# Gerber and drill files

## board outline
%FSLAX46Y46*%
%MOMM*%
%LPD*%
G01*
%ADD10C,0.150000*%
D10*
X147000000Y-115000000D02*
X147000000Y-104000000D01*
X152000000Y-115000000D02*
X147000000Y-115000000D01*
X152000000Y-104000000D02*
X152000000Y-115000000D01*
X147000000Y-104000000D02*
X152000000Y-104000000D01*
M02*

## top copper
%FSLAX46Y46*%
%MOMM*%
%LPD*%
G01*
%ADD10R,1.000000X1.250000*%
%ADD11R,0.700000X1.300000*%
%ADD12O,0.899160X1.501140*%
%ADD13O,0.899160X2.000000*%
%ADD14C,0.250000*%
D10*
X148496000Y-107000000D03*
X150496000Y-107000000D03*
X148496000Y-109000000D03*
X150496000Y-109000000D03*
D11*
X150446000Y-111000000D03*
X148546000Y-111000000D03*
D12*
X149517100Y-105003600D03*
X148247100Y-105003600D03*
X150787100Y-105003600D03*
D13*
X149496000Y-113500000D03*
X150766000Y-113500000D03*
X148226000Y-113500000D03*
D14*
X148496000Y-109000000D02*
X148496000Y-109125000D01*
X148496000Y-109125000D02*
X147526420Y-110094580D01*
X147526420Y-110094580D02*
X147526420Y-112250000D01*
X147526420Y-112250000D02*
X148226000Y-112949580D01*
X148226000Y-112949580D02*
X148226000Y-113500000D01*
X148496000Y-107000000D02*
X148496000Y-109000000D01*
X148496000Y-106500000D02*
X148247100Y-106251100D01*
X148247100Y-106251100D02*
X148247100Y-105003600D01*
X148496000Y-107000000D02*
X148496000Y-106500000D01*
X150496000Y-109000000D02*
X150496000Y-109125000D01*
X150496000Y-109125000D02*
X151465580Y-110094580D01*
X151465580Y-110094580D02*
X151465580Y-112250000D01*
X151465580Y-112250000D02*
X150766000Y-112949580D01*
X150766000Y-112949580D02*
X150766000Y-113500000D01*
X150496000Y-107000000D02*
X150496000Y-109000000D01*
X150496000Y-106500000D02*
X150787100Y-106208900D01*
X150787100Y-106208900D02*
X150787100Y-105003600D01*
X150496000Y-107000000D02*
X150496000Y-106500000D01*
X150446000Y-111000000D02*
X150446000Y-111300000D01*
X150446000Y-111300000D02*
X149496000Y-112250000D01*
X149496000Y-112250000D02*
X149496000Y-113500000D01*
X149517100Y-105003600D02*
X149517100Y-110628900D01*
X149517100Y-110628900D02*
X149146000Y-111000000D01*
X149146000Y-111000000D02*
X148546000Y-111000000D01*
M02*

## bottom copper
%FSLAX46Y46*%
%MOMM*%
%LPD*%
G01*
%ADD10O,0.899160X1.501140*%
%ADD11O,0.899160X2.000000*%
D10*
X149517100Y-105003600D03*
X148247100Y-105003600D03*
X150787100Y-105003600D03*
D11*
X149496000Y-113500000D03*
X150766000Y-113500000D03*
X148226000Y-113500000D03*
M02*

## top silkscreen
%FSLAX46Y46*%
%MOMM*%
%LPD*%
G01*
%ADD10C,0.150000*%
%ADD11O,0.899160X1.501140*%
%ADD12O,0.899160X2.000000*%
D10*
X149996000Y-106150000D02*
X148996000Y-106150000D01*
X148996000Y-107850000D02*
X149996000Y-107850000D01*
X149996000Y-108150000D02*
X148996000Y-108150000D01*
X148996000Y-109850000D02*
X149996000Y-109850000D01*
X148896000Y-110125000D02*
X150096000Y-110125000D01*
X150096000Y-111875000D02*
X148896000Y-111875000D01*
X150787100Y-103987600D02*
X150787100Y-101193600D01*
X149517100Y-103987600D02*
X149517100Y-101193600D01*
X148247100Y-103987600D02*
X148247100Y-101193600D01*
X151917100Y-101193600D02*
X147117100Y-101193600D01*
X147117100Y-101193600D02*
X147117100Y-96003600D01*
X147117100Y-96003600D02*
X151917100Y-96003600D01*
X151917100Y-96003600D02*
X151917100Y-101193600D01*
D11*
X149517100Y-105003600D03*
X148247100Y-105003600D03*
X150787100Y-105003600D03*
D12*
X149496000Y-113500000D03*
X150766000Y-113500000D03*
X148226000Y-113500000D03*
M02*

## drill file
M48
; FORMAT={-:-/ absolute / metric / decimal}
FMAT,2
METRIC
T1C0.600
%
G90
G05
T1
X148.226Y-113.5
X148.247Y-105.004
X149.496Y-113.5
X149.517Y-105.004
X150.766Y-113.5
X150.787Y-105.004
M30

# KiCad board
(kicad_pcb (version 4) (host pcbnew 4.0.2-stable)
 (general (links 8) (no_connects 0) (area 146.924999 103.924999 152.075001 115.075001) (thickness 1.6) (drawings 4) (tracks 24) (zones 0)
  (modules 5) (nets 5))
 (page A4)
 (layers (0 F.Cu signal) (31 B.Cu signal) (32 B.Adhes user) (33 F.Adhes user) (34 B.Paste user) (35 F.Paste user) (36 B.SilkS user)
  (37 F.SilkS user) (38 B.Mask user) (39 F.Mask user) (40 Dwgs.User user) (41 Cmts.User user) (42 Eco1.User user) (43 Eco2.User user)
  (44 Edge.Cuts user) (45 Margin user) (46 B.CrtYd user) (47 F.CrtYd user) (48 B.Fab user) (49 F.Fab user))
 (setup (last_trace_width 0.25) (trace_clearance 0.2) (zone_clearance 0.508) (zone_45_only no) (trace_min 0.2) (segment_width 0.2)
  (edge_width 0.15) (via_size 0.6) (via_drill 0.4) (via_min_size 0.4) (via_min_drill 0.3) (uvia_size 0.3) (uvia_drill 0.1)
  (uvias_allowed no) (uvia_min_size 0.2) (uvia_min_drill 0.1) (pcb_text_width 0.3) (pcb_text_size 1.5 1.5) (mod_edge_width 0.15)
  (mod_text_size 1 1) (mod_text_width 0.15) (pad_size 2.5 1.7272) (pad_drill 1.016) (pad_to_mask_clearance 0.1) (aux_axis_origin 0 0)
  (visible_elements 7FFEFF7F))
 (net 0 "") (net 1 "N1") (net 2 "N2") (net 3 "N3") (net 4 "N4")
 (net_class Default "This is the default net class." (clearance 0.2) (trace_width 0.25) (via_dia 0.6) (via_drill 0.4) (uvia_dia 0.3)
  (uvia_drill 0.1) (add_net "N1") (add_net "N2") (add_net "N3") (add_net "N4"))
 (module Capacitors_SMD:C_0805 (layer F.Cu) (at 149.496 107)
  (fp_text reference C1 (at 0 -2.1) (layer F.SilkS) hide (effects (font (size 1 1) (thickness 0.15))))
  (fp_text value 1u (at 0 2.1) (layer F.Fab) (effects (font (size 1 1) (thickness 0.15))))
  (fp_line (start 0.5 -0.85) (end -0.5 -0.85) (layer F.SilkS) (width 0.15))
  (fp_line (start -0.5 0.85) (end 0.5 0.85) (layer F.SilkS) (width 0.15))
  (pad 1 smd rect (at -1 0) (size 1 1.25) (layers F.Cu F.Paste F.Mask) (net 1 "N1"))
  (pad 2 smd rect (at 1 0) (size 1 1.25) (layers F.Cu F.Paste F.Mask) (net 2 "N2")))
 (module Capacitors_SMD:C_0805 (layer F.Cu) (at 149.496 109)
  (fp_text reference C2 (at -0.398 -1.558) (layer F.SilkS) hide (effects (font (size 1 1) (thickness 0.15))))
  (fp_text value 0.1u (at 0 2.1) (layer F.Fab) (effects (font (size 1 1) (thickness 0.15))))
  (fp_line (start 0.5 -0.85) (end -0.5 -0.85) (layer F.SilkS) (width 0.15))
  (fp_line (start -0.5 0.85) (end 0.5 0.85) (layer F.SilkS) (width 0.15))
  (pad 1 smd rect (at -1 0) (size 1 1.25) (layers F.Cu F.Paste F.Mask) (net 1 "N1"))
  (pad 2 smd rect (at 1 0) (size 1 1.25) (layers F.Cu F.Paste F.Mask) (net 2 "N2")))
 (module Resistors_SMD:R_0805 (layer F.Cu) (at 149.496 111 180)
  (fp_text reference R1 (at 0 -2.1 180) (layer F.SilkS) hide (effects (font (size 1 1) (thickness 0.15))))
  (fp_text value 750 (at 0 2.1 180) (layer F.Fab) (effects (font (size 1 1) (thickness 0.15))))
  (fp_line (start 0.6 0.875) (end -0.6 0.875) (layer F.SilkS) (width 0.15))
  (fp_line (start -0.6 -0.875) (end 0.6 -0.875) (layer F.SilkS) (width 0.15))
  (pad 1 smd rect (at -0.95 0 180) (size 0.7 1.3) (layers F.Cu F.Paste F.Mask) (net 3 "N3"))
  (pad 2 smd rect (at 0.95 0 180) (size 0.7 1.3) (layers F.Cu F.Paste F.Mask) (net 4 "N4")))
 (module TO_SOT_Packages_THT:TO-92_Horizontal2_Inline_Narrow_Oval (layer F.Cu) (at 148.2471 105.0036)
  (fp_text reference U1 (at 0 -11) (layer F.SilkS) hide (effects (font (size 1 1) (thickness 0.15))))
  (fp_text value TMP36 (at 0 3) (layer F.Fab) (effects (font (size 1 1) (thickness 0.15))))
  (fp_line (start 2.54 -1.016) (end 2.54 -3.81) (layer F.SilkS) (width 0.15))
  (fp_line (start 1.27 -1.016) (end 1.27 -3.81) (layer F.SilkS) (width 0.15))
  (fp_line (start 0 -1.016) (end 0 -3.81) (layer F.SilkS) (width 0.15))
  (fp_line (start 3.67 -3.81) (end -1.13 -3.81) (layer F.SilkS) (width 0.15))
  (fp_line (start -1.13 -3.81) (end -1.13 -9) (layer F.SilkS) (width 0.15))
  (fp_line (start -1.13 -9) (end 3.67 -9) (layer F.SilkS) (width 0.15))
  (fp_line (start 3.67 -9) (end 3.67 -3.81) (layer F.SilkS) (width 0.15))
  (pad 2 thru_hole oval (at 1.27 0) (size 0.89916 1.50114) (drill 0.6) (layers *.Cu *.Mask F.SilkS) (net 4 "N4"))
  (pad 1 thru_hole oval (at 0 0) (size 0.89916 1.50114) (drill 0.6) (layers *.Cu *.Mask F.SilkS) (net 1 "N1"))
  (pad 3 thru_hole oval (at 2.54 0) (size 0.89916 1.50114) (drill 0.6) (layers *.Cu *.Mask F.SilkS) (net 2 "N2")))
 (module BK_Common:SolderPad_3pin (layer F.Cu) (at 148.226 113.5)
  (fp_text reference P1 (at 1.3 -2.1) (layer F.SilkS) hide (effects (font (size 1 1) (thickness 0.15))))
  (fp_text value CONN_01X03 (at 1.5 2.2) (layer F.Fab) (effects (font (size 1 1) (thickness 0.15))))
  (pad 2 thru_hole oval (at 1.27 0 180) (size 0.89916 2) (drill 0.6) (layers *.Cu *.Mask F.SilkS) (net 3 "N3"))
  (pad 3 thru_hole oval (at 2.54 0 180) (size 0.89916 2) (drill 0.6) (layers *.Cu *.Mask F.SilkS) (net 2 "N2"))
  (pad 1 thru_hole oval (at 0 0 180) (size 0.89916 2) (drill 0.6) (layers *.Cu *.Mask F.SilkS) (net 1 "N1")))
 (gr_line (start 147 115) (end 147 104) (layer Edge.Cuts) (width 0.15))
 (gr_line (start 152 115) (end 147 115) (layer Edge.Cuts) (width 0.15))
 (gr_line (start 152 104) (end 152 115) (layer Edge.Cuts) (width 0.15))
 (gr_line (start 147 104) (end 152 104) (layer Edge.Cuts) (width 0.15))
 (segment (start 148.496 109) (end 148.496 109.125) (width 0.25) (layer F.Cu) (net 1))
 (segment (start 148.496 109.125) (end 147.52642 110.09458) (width 0.25) (layer F.Cu) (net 1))
 (segment (start 147.52642 110.09458) (end 147.52642 112.25) (width 0.25) (layer F.Cu) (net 1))
 (segment (start 147.52642 112.25) (end 148.226 112.94958) (width 0.25) (layer F.Cu) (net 1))
 (segment (start 148.226 112.94958) (end 148.226 113.5) (width 0.25) (layer F.Cu) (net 1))
 (segment (start 148.496 107) (end 148.496 109) (width 0.25) (layer F.Cu) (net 1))
 (segment (start 148.496 106.5) (end 148.2471 106.2511) (width 0.25) (layer F.Cu) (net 1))
 (segment (start 148.2471 106.2511) (end 148.2471 105.0036) (width 0.25) (layer F.Cu) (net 1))
 (segment (start 148.496 107) (end 148.496 106.5) (width 0.25) (layer F.Cu) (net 1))
 (segment (start 150.496 109) (end 150.496 109.125) (width 0.25) (layer F.Cu) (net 2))
 (segment (start 150.496 109.125) (end 151.46558 110.09458) (width 0.25) (layer F.Cu) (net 2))
 (segment (start 151.46558 110.09458) (end 151.46558 112.25) (width 0.25) (layer F.Cu) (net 2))
 (segment (start 151.46558 112.25) (end 150.766 112.94958) (width 0.25) (layer F.Cu) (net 2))
 (segment (start 150.766 112.94958) (end 150.766 113.5) (width 0.25) (layer F.Cu) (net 2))
 (segment (start 150.496 107) (end 150.496 109) (width 0.25) (layer F.Cu) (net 2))
 (segment (start 150.496 106.5) (end 150.7871 106.2089) (width 0.25) (layer F.Cu) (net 2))
 (segment (start 150.7871 106.2089) (end 150.7871 105.0036) (width 0.25) (layer F.Cu) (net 2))
 (segment (start 150.496 107) (end 150.496 106.5) (width 0.25) (layer F.Cu) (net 2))
 (segment (start 150.446 111) (end 150.446 111.3) (width 0.25) (layer F.Cu) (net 3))
 (segment (start 150.446 111.3) (end 149.496 112.25) (width 0.25) (layer F.Cu) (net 3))
 (segment (start 149.496 112.25) (end 149.496 113.5) (width 0.25) (layer F.Cu) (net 3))
 (segment (start 149.5171 105.0036) (end 149.5171 110.6289) (width 0.25) (layer F.Cu) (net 4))
 (segment (start 149.5171 110.6289) (end 149.146 111) (width 0.25) (layer F.Cu) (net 4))
 (segment (start 149.146 111) (end 148.546 111) (width 0.25) (layer F.Cu) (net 4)))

